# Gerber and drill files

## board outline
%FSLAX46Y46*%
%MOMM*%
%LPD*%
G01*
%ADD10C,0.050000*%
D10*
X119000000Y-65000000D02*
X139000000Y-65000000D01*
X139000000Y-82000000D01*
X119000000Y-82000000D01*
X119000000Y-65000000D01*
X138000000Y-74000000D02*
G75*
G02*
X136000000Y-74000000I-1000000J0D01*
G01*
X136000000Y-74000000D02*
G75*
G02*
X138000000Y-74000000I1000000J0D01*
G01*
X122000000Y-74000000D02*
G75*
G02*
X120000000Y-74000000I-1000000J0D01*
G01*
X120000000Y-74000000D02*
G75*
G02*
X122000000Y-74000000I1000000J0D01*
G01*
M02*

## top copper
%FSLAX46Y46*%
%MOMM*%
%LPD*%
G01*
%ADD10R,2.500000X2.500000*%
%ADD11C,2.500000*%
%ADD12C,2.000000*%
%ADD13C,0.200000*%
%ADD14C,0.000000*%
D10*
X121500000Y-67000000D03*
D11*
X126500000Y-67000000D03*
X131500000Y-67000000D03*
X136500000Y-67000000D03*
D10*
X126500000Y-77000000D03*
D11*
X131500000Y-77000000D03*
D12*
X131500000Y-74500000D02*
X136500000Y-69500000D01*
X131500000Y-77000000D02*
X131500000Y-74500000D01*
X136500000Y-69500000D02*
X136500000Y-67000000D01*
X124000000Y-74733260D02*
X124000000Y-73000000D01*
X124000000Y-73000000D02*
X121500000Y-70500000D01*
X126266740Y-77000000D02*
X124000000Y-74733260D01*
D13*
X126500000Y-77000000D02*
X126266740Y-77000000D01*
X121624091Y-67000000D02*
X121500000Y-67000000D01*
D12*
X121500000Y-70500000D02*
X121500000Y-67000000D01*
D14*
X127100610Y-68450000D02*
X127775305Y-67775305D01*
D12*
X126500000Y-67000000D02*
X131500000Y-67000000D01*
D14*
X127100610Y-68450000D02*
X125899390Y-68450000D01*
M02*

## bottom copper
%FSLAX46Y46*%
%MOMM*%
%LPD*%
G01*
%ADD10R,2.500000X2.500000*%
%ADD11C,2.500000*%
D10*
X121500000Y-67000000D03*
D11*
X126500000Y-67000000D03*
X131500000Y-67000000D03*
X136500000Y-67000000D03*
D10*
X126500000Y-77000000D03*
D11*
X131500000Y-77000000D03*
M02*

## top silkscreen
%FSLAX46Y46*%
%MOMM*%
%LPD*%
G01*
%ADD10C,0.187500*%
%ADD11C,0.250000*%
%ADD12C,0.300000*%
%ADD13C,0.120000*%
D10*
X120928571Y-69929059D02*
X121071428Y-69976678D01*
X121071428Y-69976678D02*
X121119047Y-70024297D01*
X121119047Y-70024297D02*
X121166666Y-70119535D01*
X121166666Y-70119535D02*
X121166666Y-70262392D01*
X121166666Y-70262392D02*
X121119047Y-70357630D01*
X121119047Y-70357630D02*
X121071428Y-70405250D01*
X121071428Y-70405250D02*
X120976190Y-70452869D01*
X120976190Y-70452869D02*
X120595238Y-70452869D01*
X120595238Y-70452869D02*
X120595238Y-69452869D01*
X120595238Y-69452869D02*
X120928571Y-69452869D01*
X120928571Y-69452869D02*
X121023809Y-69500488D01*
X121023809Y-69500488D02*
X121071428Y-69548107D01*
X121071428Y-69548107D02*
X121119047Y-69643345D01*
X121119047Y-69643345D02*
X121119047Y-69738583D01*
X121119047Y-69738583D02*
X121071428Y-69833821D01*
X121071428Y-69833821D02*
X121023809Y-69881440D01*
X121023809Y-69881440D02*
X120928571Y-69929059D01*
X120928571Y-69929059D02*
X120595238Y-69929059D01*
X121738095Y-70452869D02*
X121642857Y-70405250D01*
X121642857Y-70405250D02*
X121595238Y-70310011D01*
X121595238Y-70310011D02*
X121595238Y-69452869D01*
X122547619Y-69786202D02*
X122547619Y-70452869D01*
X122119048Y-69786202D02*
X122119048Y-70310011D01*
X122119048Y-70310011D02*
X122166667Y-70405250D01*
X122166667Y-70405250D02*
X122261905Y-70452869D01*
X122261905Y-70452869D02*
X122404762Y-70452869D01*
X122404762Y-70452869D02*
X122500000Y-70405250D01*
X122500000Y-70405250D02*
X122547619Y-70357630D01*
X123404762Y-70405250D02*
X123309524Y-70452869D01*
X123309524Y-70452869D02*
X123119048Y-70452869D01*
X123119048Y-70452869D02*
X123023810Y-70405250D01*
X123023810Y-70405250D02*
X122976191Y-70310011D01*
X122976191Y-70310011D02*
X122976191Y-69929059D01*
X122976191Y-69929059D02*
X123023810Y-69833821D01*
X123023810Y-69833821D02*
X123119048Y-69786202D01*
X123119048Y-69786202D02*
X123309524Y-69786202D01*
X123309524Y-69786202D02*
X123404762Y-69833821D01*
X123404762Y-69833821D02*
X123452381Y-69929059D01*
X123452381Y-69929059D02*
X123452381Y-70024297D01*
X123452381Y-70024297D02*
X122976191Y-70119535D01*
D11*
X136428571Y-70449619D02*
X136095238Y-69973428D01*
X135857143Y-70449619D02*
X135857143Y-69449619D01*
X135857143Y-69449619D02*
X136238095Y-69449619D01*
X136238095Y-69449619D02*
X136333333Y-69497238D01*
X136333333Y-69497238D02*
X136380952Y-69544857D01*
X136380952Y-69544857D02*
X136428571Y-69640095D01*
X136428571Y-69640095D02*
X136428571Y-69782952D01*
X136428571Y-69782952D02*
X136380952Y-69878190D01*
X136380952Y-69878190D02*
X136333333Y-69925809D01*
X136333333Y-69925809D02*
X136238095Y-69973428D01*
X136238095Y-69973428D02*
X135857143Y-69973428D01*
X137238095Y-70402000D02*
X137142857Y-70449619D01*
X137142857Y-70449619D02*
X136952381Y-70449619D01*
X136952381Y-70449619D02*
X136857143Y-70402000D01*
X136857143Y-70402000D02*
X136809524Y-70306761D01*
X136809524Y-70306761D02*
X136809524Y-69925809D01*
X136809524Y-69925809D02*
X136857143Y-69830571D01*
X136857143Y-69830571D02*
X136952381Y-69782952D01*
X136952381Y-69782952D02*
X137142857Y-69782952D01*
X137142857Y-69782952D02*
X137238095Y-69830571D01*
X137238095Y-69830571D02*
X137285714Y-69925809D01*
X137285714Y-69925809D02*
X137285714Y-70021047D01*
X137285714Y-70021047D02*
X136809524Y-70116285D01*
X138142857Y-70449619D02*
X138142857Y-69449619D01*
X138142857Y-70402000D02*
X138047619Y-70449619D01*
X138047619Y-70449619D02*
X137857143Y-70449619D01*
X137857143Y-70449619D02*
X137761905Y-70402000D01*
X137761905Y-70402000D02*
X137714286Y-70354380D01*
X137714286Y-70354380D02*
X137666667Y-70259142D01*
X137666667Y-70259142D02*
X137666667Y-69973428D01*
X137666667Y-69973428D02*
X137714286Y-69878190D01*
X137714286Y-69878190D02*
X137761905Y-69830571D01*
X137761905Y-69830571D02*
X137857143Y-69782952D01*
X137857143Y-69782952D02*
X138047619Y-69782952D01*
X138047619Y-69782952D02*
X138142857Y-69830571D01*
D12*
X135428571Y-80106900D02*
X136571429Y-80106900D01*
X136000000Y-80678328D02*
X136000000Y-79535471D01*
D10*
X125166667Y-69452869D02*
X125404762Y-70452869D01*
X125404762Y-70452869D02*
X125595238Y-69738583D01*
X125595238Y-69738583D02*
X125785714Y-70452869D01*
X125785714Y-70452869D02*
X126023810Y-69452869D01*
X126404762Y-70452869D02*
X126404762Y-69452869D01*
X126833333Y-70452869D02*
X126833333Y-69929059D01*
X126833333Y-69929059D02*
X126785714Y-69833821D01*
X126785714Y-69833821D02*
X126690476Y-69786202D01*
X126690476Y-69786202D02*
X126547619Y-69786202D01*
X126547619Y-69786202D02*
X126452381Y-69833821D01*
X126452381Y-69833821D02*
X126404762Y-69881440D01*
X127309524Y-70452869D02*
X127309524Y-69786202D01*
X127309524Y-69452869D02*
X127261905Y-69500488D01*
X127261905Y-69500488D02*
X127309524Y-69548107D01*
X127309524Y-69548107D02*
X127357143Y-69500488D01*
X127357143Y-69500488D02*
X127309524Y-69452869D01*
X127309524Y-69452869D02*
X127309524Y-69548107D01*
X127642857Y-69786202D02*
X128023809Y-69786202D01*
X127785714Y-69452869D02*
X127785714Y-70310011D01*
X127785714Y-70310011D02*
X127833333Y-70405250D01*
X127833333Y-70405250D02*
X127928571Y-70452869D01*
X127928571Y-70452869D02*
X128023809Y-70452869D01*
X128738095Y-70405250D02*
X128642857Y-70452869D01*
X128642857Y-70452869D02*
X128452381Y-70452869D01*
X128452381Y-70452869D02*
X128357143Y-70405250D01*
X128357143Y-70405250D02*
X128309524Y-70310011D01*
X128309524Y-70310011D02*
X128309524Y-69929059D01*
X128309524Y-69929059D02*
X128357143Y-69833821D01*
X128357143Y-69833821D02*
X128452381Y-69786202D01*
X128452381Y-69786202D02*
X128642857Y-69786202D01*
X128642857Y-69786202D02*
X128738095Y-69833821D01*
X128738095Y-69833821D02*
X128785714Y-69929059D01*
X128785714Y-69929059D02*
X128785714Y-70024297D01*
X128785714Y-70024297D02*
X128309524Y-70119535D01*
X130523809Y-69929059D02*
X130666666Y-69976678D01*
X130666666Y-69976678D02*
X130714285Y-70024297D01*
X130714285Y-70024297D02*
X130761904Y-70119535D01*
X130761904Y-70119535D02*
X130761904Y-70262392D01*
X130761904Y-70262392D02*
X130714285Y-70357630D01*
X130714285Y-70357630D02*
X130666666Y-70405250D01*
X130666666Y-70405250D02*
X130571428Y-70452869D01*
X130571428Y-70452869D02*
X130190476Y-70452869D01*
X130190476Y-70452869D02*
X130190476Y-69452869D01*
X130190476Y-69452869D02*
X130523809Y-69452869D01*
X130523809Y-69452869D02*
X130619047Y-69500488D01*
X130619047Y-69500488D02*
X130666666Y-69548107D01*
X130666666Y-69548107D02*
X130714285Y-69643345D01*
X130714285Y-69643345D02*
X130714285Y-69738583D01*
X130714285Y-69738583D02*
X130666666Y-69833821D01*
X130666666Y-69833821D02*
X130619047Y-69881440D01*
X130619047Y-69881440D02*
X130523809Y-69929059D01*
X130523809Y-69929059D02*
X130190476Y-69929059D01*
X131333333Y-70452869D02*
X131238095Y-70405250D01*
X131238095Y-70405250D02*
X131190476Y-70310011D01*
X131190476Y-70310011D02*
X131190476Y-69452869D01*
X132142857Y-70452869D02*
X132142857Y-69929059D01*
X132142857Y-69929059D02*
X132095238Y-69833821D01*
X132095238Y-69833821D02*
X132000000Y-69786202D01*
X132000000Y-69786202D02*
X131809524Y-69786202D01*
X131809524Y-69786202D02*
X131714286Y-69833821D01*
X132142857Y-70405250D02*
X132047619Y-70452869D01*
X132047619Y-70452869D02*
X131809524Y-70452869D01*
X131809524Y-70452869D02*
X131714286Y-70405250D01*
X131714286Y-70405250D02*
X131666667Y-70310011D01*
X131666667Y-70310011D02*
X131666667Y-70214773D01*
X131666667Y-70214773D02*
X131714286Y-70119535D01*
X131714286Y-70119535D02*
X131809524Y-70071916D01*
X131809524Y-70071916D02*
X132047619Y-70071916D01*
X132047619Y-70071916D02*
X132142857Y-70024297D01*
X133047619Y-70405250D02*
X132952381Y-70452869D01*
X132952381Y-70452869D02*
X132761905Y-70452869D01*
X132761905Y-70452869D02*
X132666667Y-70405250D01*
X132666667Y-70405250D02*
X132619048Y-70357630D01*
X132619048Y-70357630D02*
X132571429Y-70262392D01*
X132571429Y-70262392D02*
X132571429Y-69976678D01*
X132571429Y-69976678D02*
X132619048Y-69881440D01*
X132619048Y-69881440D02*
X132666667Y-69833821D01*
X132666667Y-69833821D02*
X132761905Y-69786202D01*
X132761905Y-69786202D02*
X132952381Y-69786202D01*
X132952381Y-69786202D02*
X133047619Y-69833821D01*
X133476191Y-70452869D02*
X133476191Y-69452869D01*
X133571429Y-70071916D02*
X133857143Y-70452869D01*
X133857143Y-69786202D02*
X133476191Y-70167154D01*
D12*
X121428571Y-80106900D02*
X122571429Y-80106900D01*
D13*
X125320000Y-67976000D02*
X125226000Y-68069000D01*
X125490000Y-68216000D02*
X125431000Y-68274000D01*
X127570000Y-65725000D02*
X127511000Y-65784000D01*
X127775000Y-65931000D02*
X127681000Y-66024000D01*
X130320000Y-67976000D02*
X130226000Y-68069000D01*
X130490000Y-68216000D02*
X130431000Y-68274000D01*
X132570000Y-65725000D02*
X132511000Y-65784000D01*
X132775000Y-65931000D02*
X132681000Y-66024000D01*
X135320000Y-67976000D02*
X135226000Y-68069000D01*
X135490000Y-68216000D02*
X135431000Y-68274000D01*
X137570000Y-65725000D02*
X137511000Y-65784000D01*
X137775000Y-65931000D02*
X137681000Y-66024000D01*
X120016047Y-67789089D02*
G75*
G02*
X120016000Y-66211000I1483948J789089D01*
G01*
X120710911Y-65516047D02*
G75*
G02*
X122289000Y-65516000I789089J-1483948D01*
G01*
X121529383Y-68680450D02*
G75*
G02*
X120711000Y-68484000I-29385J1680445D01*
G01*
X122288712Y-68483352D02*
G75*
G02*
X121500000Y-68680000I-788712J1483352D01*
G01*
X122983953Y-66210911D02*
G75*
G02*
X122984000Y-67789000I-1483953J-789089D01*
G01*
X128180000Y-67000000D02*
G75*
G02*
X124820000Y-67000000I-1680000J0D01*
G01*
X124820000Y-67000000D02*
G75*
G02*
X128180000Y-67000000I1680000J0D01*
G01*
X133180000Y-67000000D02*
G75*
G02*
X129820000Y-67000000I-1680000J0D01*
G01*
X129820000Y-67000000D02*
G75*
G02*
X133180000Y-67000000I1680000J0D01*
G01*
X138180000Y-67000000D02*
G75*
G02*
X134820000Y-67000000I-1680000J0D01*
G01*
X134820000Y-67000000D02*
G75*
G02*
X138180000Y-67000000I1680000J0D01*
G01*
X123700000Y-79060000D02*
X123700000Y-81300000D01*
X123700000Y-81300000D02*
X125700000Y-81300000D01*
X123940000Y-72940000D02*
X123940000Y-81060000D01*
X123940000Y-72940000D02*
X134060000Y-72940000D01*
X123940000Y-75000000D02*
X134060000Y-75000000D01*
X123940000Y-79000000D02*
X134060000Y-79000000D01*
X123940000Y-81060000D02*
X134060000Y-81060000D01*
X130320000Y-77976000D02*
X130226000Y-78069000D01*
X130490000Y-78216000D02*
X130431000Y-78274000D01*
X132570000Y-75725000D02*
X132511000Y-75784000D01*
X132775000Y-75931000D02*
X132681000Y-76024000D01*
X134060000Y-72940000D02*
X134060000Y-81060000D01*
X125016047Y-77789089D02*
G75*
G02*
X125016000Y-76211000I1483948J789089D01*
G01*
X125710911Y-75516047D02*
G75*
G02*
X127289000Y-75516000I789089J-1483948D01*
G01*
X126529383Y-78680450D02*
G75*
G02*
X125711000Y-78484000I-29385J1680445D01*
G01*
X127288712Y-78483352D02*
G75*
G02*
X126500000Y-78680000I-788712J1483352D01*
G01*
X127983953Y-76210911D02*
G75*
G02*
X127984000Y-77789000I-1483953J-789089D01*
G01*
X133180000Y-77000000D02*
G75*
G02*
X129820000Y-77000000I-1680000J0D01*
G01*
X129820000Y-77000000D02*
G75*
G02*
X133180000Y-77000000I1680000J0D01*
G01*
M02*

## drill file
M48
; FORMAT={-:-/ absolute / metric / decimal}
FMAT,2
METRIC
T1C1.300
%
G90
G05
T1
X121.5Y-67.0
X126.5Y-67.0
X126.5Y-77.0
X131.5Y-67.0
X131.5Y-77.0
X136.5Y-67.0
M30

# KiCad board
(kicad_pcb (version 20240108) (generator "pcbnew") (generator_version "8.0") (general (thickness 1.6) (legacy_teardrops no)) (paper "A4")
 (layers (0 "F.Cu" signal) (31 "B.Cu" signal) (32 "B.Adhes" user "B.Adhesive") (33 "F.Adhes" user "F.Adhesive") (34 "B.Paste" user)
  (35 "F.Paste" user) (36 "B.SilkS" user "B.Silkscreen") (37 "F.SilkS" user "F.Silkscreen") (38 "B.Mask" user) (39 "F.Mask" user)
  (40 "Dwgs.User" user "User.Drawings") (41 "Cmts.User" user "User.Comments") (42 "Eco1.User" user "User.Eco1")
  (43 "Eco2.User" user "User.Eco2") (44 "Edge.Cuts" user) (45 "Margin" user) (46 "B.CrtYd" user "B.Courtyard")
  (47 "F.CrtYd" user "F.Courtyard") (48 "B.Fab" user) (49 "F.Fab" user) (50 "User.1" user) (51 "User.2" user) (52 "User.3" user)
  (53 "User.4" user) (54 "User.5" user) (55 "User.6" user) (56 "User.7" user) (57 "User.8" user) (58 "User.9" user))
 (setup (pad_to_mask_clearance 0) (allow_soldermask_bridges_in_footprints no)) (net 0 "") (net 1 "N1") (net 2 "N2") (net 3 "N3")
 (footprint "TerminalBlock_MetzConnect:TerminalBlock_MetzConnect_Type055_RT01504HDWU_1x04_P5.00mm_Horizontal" (layer "F.Cu") (at 121.5 67)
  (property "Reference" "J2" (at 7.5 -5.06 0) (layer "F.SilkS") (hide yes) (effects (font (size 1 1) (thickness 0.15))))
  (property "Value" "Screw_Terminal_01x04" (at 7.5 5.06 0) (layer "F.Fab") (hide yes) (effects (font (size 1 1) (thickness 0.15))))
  (fp_line (start 3.82 0.976) (end 3.726 1.069) (stroke (width 0.12) (type solid)) (layer "F.SilkS"))
  (fp_line (start 3.99 1.216) (end 3.931 1.274) (stroke (width 0.12) (type solid)) (layer "F.SilkS"))
  (fp_line (start 6.07 -1.275) (end 6.011 -1.216) (stroke (width 0.12) (type solid)) (layer "F.SilkS"))
  (fp_line (start 6.275 -1.069) (end 6.181 -0.976) (stroke (width 0.12) (type solid)) (layer "F.SilkS"))
  (fp_line (start 8.82 0.976) (end 8.726 1.069) (stroke (width 0.12) (type solid)) (layer "F.SilkS"))
  (fp_line (start 8.99 1.216) (end 8.931 1.274) (stroke (width 0.12) (type solid)) (layer "F.SilkS"))
  (fp_line (start 11.07 -1.275) (end 11.011 -1.216) (stroke (width 0.12) (type solid)) (layer "F.SilkS"))
  (fp_line (start 11.275 -1.069) (end 11.181 -0.976) (stroke (width 0.12) (type solid)) (layer "F.SilkS"))
  (fp_line (start 13.82 0.976) (end 13.726 1.069) (stroke (width 0.12) (type solid)) (layer "F.SilkS"))
  (fp_line (start 13.99 1.216) (end 13.931 1.274) (stroke (width 0.12) (type solid)) (layer "F.SilkS"))
  (fp_line (start 16.07 -1.275) (end 16.011 -1.216) (stroke (width 0.12) (type solid)) (layer "F.SilkS"))
  (fp_line (start 16.275 -1.069) (end 16.181 -0.976) (stroke (width 0.12) (type solid)) (layer "F.SilkS"))
  (fp_arc (start -1.483953 0.789089) (mid -1.680708 0.00005) (end -1.484 -0.789) (stroke (width 0.12) (type solid)) (layer "F.SilkS"))
  (fp_arc (start -0.789089 -1.483953) (mid -0.00005 -1.680708) (end 0.789 -1.484) (stroke (width 0.12) (type solid)) (layer "F.SilkS"))
  (fp_arc (start 0.029383 1.68045) (mid -0.392304 1.634281) (end -0.789 1.484) (stroke (width 0.12) (type solid)) (layer "F.SilkS"))
  (fp_arc (start 0.788712 1.483352) (mid 0.406429 1.630097) (end 0 1.68) (stroke (width 0.12) (type solid)) (layer "F.SilkS"))
  (fp_arc (start 1.483953 -0.789089) (mid 1.680708 -0.00005) (end 1.484 0.789) (stroke (width 0.12) (type solid)) (layer "F.SilkS"))
  (fp_circle (center 5 0) (end 6.68 0) (stroke (width 0.12) (type solid)) (fill none) (layer "F.SilkS"))
  (fp_circle (center 10 0) (end 11.68 0) (stroke (width 0.12) (type solid)) (fill none) (layer "F.SilkS"))
  (fp_circle (center 15 0) (end 16.68 0) (stroke (width 0.12) (type solid)) (fill none) (layer "F.SilkS"))
  (pad "1" thru_hole rect (at 0 0) (size 2.5 2.5) (drill 1.3) (layers "*.Cu" "*.Mask") (remove_unused_layers no) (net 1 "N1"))
  (pad "2" thru_hole circle (at 5 0) (size 2.5 2.5) (drill 1.3) (layers "*.Cu" "*.Mask") (remove_unused_layers no) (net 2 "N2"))
  (pad "3" thru_hole circle (at 10 0) (size 2.5 2.5) (drill 1.3) (layers "*.Cu" "*.Mask") (remove_unused_layers no) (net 2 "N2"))
  (pad "4" thru_hole circle (at 15 0) (size 2.5 2.5) (drill 1.3) (layers "*.Cu" "*.Mask") (remove_unused_layers no) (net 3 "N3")))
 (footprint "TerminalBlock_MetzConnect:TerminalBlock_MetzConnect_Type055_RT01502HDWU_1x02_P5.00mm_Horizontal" (layer "F.Cu") (at 126.5 77)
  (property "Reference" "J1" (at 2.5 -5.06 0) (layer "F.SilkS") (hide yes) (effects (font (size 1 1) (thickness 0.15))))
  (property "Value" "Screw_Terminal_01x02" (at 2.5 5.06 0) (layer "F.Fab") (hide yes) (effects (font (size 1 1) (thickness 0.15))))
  (fp_line (start -2.8 2.06) (end -2.8 4.3) (stroke (width 0.12) (type solid)) (layer "F.SilkS"))
  (fp_line (start -2.8 4.3) (end -0.8 4.3) (stroke (width 0.12) (type solid)) (layer "F.SilkS"))
  (fp_line (start -2.56 -4.06) (end -2.56 4.06) (stroke (width 0.12) (type solid)) (layer "F.SilkS"))
  (fp_line (start -2.56 -4.06) (end 7.56 -4.06) (stroke (width 0.12) (type solid)) (layer "F.SilkS"))
  (fp_line (start -2.56 -2) (end 7.56 -2) (stroke (width 0.12) (type solid)) (layer "F.SilkS"))
  (fp_line (start -2.56 2) (end 7.56 2) (stroke (width 0.12) (type solid)) (layer "F.SilkS"))
  (fp_line (start -2.56 4.06) (end 7.56 4.06) (stroke (width 0.12) (type solid)) (layer "F.SilkS"))
  (fp_line (start 3.82 0.976) (end 3.726 1.069) (stroke (width 0.12) (type solid)) (layer "F.SilkS"))
  (fp_line (start 3.99 1.216) (end 3.931 1.274) (stroke (width 0.12) (type solid)) (layer "F.SilkS"))
  (fp_line (start 6.07 -1.275) (end 6.011 -1.216) (stroke (width 0.12) (type solid)) (layer "F.SilkS"))
  (fp_line (start 6.275 -1.069) (end 6.181 -0.976) (stroke (width 0.12) (type solid)) (layer "F.SilkS"))
  (fp_line (start 7.56 -4.06) (end 7.56 4.06) (stroke (width 0.12) (type solid)) (layer "F.SilkS"))
  (fp_arc (start -1.483953 0.789089) (mid -1.680708 0.00005) (end -1.484 -0.789) (stroke (width 0.12) (type solid)) (layer "F.SilkS"))
  (fp_arc (start -0.789089 -1.483953) (mid -0.00005 -1.680708) (end 0.789 -1.484) (stroke (width 0.12) (type solid)) (layer "F.SilkS"))
  (fp_arc (start 0.029383 1.68045) (mid -0.392304 1.634281) (end -0.789 1.484) (stroke (width 0.12) (type solid)) (layer "F.SilkS"))
  (fp_arc (start 0.788712 1.483352) (mid 0.406429 1.630097) (end 0 1.68) (stroke (width 0.12) (type solid)) (layer "F.SilkS"))
  (fp_arc (start 1.483953 -0.789089) (mid 1.680708 -0.00005) (end 1.484 0.789) (stroke (width 0.12) (type solid)) (layer "F.SilkS"))
  (fp_circle (center 5 0) (end 6.68 0) (stroke (width 0.12) (type solid)) (fill none) (layer "F.SilkS"))
  (pad "1" thru_hole rect (at 0 0) (size 2.5 2.5) (drill 1.3) (layers "*.Cu" "*.Mask") (remove_unused_layers no) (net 1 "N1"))
  (pad "2" thru_hole circle (at 5 0) (size 2.5 2.5) (drill 1.3) (layers "*.Cu" "*.Mask") (remove_unused_layers no) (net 3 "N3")))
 (gr_rect (start 119 65) (end 139 82) (stroke (width 0.05) (type default)) (fill none) (layer "Edge.Cuts"))
 (gr_circle (center 137 74) (end 138 74) (stroke (width 0.05) (type default)) (fill none) (layer "Edge.Cuts"))
 (gr_circle (center 121 74) (end 122 74) (stroke (width 0.05) (type default)) (fill none) (layer "Edge.Cuts"))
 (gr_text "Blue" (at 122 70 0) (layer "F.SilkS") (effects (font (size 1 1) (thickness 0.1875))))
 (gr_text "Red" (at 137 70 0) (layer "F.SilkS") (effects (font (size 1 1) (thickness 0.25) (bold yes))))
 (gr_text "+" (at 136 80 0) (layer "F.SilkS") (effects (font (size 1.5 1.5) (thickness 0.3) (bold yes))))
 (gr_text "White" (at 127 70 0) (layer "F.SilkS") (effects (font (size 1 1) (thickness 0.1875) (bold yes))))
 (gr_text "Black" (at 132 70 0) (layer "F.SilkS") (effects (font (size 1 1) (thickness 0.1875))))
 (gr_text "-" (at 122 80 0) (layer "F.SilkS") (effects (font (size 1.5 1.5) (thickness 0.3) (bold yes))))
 (segment (start 131.5 74.5) (end 136.5 69.5) (width 2) (layer "F.Cu") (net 3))
 (segment (start 131.5 77) (end 131.5 74.5) (width 2) (layer "F.Cu") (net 3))
 (segment (start 136.5 69.5) (end 136.5 67) (width 2) (layer "F.Cu") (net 3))
 (segment (start 124 74.73326) (end 124 73) (width 2) (layer "F.Cu") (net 1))
 (segment (start 124 73) (end 121.5 70.5) (width 2) (layer "F.Cu") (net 1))
 (segment (start 126.26674 77) (end 124 74.73326) (width 2) (layer "F.Cu") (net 1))
 (segment (start 126.5 77) (end 126.26674 77) (width 0.2) (layer "F.Cu") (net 1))
 (segment (start 121.624091 67) (end 121.5 67) (width 0.2) (layer "F.Cu") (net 1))
 (segment (start 121.5 70.5) (end 121.5 67) (width 2) (layer "F.Cu") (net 1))
 (segment (start 127.10061 68.45) (end 127.775305 67.775305) (width 0) (layer "F.Cu") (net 2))
 (segment (start 126.5 67) (end 131.5 67) (width 2) (layer "F.Cu") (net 2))
 (segment (start 127.10061 68.45) (end 125.89939 68.45) (width 0) (layer "F.Cu") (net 2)))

